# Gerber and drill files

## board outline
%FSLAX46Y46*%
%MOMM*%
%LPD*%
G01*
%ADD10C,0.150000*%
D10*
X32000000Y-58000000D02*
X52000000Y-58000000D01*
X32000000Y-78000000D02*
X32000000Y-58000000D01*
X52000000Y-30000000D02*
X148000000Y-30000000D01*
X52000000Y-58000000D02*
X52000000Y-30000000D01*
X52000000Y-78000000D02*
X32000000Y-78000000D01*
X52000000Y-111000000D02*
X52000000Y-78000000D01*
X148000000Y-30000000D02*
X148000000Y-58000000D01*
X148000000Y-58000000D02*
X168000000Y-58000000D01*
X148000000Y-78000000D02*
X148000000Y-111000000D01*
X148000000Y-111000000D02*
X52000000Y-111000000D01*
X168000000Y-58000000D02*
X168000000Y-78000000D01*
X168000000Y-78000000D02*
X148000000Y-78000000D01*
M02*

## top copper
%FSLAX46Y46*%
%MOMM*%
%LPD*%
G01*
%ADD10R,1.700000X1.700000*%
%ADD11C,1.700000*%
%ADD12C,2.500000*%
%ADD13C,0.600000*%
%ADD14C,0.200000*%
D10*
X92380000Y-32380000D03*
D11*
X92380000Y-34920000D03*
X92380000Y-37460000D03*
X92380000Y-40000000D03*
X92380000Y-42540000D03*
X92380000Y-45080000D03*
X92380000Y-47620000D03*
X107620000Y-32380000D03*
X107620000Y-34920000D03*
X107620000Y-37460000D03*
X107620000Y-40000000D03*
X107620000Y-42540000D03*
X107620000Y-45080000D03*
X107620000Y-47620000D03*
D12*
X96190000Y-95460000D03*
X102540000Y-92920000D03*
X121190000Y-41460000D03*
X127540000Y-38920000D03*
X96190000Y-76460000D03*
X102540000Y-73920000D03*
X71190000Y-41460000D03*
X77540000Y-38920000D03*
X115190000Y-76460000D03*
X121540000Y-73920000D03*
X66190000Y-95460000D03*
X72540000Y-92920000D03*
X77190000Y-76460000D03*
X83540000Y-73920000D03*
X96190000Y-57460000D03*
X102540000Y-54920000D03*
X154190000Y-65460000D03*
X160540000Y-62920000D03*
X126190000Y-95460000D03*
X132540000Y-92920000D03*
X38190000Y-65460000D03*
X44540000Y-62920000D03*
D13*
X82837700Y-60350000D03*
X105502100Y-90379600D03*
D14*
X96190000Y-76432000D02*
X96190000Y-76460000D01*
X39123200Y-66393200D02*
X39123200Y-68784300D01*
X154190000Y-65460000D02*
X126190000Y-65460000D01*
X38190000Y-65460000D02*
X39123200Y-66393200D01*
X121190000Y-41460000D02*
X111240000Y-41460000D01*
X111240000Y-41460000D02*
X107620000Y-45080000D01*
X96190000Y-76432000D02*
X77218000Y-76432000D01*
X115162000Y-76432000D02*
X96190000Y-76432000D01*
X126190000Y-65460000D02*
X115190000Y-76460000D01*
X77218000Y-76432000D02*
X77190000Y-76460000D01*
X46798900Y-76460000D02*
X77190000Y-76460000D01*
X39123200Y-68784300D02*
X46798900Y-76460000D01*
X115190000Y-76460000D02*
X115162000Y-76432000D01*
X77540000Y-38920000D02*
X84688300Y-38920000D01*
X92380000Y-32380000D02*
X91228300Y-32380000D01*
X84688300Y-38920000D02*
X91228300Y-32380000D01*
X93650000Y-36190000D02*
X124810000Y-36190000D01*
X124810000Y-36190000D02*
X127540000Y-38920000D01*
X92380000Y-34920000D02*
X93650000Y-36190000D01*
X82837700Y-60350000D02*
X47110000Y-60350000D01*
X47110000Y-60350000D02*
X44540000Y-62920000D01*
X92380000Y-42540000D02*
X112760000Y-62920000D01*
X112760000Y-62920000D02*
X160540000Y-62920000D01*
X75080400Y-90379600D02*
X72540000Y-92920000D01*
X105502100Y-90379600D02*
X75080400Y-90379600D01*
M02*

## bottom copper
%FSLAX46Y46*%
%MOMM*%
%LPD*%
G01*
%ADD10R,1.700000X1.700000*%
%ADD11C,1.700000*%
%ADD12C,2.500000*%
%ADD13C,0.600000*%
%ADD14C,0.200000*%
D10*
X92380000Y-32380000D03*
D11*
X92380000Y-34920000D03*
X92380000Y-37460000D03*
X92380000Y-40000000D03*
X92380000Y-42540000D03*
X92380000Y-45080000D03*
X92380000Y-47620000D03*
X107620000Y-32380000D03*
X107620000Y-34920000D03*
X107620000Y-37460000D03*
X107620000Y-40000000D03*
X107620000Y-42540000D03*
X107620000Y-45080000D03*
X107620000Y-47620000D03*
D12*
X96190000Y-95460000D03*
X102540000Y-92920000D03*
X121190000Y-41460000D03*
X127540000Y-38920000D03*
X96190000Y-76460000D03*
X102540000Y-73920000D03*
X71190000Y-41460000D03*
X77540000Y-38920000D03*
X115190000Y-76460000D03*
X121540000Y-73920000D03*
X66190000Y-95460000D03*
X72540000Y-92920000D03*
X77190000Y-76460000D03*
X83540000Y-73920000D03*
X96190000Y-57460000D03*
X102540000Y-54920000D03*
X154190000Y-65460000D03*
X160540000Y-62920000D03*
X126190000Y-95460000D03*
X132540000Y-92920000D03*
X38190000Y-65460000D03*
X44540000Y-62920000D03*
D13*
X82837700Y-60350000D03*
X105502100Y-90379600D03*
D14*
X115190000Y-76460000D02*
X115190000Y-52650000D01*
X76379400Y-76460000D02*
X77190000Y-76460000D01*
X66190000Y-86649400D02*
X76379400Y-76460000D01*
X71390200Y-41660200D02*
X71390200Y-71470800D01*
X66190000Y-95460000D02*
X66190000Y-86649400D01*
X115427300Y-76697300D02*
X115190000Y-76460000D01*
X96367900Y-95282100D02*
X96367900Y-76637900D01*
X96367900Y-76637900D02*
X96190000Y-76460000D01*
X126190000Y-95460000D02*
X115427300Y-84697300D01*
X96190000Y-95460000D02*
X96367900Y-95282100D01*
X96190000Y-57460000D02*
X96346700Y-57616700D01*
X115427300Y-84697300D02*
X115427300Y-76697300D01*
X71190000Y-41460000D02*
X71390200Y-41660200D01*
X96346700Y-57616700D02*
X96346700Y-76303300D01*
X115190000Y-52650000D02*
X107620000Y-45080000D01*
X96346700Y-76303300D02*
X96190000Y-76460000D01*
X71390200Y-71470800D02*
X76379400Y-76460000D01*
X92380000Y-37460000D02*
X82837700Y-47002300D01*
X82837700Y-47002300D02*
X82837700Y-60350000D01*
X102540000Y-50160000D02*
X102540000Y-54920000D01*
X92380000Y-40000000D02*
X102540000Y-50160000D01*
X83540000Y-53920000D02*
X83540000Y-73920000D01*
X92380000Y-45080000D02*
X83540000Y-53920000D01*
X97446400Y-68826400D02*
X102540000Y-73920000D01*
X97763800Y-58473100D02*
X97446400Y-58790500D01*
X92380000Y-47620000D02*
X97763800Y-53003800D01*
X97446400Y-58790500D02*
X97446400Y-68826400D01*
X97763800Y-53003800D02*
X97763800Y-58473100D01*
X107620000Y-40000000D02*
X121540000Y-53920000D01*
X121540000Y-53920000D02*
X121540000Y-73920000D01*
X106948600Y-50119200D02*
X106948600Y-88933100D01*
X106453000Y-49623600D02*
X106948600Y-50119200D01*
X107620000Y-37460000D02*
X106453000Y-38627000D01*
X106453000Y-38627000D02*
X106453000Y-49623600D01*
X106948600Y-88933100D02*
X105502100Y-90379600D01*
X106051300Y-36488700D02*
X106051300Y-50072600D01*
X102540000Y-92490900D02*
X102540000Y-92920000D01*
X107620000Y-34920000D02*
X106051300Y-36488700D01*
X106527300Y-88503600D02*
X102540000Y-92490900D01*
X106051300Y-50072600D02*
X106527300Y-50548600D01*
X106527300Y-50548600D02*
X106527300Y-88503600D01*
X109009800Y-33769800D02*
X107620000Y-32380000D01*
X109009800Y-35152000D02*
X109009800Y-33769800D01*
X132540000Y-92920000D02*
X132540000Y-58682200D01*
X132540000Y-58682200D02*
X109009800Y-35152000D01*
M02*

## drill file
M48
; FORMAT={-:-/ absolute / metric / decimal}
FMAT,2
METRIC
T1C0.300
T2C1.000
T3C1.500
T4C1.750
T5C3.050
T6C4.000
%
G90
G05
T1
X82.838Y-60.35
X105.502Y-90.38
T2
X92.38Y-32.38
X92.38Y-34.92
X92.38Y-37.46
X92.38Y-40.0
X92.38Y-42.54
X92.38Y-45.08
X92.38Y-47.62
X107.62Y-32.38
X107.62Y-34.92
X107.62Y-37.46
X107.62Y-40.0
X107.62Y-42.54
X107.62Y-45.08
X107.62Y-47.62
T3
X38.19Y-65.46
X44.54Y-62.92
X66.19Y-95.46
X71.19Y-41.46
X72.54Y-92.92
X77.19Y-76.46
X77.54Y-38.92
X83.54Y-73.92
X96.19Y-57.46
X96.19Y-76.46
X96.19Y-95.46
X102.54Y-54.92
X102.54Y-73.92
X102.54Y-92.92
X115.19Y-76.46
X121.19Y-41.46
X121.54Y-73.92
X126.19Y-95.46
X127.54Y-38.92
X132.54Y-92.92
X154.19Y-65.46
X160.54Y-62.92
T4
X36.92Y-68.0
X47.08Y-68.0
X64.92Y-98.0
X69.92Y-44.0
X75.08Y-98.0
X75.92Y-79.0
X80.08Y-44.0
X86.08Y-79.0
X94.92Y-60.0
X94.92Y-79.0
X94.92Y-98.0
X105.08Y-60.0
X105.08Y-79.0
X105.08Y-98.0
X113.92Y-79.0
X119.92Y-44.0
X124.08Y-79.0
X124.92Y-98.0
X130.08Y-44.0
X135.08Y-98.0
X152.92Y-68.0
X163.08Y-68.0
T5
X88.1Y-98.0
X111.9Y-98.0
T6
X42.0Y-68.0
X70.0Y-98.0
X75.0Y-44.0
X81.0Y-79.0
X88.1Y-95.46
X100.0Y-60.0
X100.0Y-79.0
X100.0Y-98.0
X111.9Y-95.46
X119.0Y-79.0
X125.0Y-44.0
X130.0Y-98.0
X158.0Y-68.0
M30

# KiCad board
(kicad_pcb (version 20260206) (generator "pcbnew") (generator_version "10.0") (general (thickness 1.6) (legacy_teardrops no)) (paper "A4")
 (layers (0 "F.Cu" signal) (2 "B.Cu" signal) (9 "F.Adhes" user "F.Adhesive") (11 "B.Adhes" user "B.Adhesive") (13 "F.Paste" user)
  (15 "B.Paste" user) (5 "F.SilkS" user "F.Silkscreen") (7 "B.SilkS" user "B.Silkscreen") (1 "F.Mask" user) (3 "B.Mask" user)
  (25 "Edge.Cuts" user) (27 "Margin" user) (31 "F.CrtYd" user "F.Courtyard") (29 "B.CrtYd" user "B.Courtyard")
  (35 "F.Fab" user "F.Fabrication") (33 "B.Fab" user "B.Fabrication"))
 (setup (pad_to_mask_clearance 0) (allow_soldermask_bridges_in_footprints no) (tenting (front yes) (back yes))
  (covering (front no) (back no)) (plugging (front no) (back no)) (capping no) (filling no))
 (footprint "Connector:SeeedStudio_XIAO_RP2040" (layer "F.Cu") (at 100 40)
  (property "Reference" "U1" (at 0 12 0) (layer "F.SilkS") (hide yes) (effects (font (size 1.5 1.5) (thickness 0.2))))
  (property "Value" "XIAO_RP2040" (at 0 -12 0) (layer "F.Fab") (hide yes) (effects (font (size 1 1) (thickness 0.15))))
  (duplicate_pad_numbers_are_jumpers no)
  (pad "1" thru_hole rect (at -7.62 -7.62) (size 1.7 1.7) (drill 1) (layers "*.Cu" "*.Mask") (remove_unused_layers no) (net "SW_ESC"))
  (pad "2" thru_hole circle (at -7.62 -5.08) (size 1.7 1.7) (drill 1) (layers "*.Cu" "*.Mask") (remove_unused_layers no) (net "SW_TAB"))
  (pad "3" thru_hole circle (at -7.62 -2.54) (size 1.7 1.7) (drill 1) (layers "*.Cu" "*.Mask") (remove_unused_layers no)
   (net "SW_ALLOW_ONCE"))
  (pad "4" thru_hole circle (at -7.62 0) (size 1.7 1.7) (drill 1) (layers "*.Cu" "*.Mask") (remove_unused_layers no) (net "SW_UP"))
  (pad "5" thru_hole circle (at -7.62 2.54) (size 1.7 1.7) (drill 1) (layers "*.Cu" "*.Mask") (remove_unused_layers no)
   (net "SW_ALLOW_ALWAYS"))
  (pad "6" thru_hole circle (at -7.62 5.08) (size 1.7 1.7) (drill 1) (layers "*.Cu" "*.Mask") (remove_unused_layers no) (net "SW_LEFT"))
  (pad "7" thru_hole circle (at -7.62 7.62) (size 1.7 1.7) (drill 1) (layers "*.Cu" "*.Mask") (remove_unused_layers no) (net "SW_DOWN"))
  (pad "8" thru_hole circle (at 7.62 -7.62) (size 1.7 1.7) (drill 1) (layers "*.Cu" "*.Mask") (remove_unused_layers no) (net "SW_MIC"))
  (pad "9" thru_hole circle (at 7.62 -5.08) (size 1.7 1.7) (drill 1) (layers "*.Cu" "*.Mask") (remove_unused_layers no) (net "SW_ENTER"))
  (pad "10" thru_hole circle (at 7.62 -2.54) (size 1.7 1.7) (drill 1) (layers "*.Cu" "*.Mask") (remove_unused_layers no) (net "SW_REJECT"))
  (pad "11" thru_hole circle (at 7.62 0) (size 1.7 1.7) (drill 1) (layers "*.Cu" "*.Mask") (remove_unused_layers no) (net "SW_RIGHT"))
  (pad "12" thru_hole circle (at 7.62 2.54) (size 1.7 1.7) (drill 1) (layers "*.Cu" "*.Mask") (remove_unused_layers no))
  (pad "13" thru_hole circle (at 7.62 5.08) (size 1.7 1.7) (drill 1) (layers "*.Cu" "*.Mask") (remove_unused_layers no) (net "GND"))
  (pad "14" thru_hole circle (at 7.62 7.62) (size 1.7 1.7) (drill 1) (layers "*.Cu" "*.Mask") (remove_unused_layers no)))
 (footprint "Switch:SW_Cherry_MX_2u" (layer "F.Cu") (at 100 98)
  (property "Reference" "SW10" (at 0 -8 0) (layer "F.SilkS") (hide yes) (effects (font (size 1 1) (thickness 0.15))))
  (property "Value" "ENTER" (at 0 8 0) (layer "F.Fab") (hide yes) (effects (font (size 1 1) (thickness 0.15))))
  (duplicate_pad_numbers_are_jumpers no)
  (pad "" np_thru_hole circle (at -11.9 -2.54) (size 4 4) (drill 4) (layers "*.Cu" "*.Mask"))
  (pad "" np_thru_hole circle (at -11.9 0) (size 3.05 3.05) (drill 3.05) (layers "*.Cu" "*.Mask"))
  (pad "" np_thru_hole circle (at -5.08 0) (size 1.75 1.75) (drill 1.75) (layers "*.Cu" "*.Mask"))
  (pad "" np_thru_hole circle (at 0 0) (size 4 4) (drill 4) (layers "*.Cu" "*.Mask"))
  (pad "" np_thru_hole circle (at 5.08 0) (size 1.75 1.75) (drill 1.75) (layers "*.Cu" "*.Mask"))
  (pad "" np_thru_hole circle (at 11.9 -2.54) (size 4 4) (drill 4) (layers "*.Cu" "*.Mask"))
  (pad "" np_thru_hole circle (at 11.9 0) (size 3.05 3.05) (drill 3.05) (layers "*.Cu" "*.Mask"))
  (pad "1" thru_hole circle (at -3.81 -2.54) (size 2.5 2.5) (drill 1.5) (layers "*.Cu" "*.Mask") (remove_unused_layers no) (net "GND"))
  (pad "2" thru_hole circle (at 2.54 -5.08) (size 2.5 2.5) (drill 1.5) (layers "*.Cu" "*.Mask") (remove_unused_layers no) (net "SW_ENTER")))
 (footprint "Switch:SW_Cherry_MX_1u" (layer "F.Cu") (at 125 44)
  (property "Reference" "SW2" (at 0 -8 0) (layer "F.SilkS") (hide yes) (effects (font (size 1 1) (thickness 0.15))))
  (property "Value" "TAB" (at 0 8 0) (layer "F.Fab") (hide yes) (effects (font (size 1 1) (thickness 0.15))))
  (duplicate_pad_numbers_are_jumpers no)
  (pad "" np_thru_hole circle (at -5.08 0) (size 1.75 1.75) (drill 1.75) (layers "*.Cu" "*.Mask"))
  (pad "" np_thru_hole circle (at 0 0) (size 4 4) (drill 4) (layers "*.Cu" "*.Mask"))
  (pad "" np_thru_hole circle (at 5.08 0) (size 1.75 1.75) (drill 1.75) (layers "*.Cu" "*.Mask"))
  (pad "1" thru_hole circle (at -3.81 -2.54) (size 2.5 2.5) (drill 1.5) (layers "*.Cu" "*.Mask") (remove_unused_layers no) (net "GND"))
  (pad "2" thru_hole circle (at 2.54 -5.08) (size 2.5 2.5) (drill 1.5) (layers "*.Cu" "*.Mask") (remove_unused_layers no) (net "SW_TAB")))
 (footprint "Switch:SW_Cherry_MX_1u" (layer "F.Cu") (at 100 79)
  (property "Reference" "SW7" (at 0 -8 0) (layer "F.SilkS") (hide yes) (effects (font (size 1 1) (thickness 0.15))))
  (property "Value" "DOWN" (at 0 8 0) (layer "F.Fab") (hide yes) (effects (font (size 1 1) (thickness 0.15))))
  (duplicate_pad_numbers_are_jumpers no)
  (pad "" np_thru_hole circle (at -5.08 0) (size 1.75 1.75) (drill 1.75) (layers "*.Cu" "*.Mask"))
  (pad "" np_thru_hole circle (at 0 0) (size 4 4) (drill 4) (layers "*.Cu" "*.Mask"))
  (pad "" np_thru_hole circle (at 5.08 0) (size 1.75 1.75) (drill 1.75) (layers "*.Cu" "*.Mask"))
  (pad "1" thru_hole circle (at -3.81 -2.54) (size 2.5 2.5) (drill 1.5) (layers "*.Cu" "*.Mask") (remove_unused_layers no) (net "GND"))
  (pad "2" thru_hole circle (at 2.54 -5.08) (size 2.5 2.5) (drill 1.5) (layers "*.Cu" "*.Mask") (remove_unused_layers no) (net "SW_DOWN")))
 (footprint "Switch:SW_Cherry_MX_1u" (layer "F.Cu") (at 75 44)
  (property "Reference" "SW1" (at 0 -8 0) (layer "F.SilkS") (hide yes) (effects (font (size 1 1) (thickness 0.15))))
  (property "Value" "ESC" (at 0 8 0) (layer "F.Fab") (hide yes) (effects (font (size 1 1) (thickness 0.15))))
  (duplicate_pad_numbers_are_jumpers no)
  (pad "" np_thru_hole circle (at -5.08 0) (size 1.75 1.75) (drill 1.75) (layers "*.Cu" "*.Mask"))
  (pad "" np_thru_hole circle (at 0 0) (size 4 4) (drill 4) (layers "*.Cu" "*.Mask"))
  (pad "" np_thru_hole circle (at 5.08 0) (size 1.75 1.75) (drill 1.75) (layers "*.Cu" "*.Mask"))
  (pad "1" thru_hole circle (at -3.81 -2.54) (size 2.5 2.5) (drill 1.5) (layers "*.Cu" "*.Mask") (remove_unused_layers no) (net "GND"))
  (pad "2" thru_hole circle (at 2.54 -5.08) (size 2.5 2.5) (drill 1.5) (layers "*.Cu" "*.Mask") (remove_unused_layers no) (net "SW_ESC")))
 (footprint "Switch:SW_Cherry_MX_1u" (layer "F.Cu") (at 119 79)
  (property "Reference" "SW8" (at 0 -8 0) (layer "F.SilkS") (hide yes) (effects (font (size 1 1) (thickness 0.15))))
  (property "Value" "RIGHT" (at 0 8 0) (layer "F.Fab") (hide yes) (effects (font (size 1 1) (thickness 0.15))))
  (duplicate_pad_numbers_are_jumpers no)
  (pad "" np_thru_hole circle (at -5.08 0) (size 1.75 1.75) (drill 1.75) (layers "*.Cu" "*.Mask"))
  (pad "" np_thru_hole circle (at 0 0) (size 4 4) (drill 4) (layers "*.Cu" "*.Mask"))
  (pad "" np_thru_hole circle (at 5.08 0) (size 1.75 1.75) (drill 1.75) (layers "*.Cu" "*.Mask"))
  (pad "1" thru_hole circle (at -3.81 -2.54) (size 2.5 2.5) (drill 1.5) (layers "*.Cu" "*.Mask") (remove_unused_layers no) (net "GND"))
  (pad "2" thru_hole circle (at 2.54 -5.08) (size 2.5 2.5) (drill 1.5) (layers "*.Cu" "*.Mask") (remove_unused_layers no) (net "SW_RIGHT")))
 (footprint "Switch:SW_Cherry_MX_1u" (layer "F.Cu") (at 70 98)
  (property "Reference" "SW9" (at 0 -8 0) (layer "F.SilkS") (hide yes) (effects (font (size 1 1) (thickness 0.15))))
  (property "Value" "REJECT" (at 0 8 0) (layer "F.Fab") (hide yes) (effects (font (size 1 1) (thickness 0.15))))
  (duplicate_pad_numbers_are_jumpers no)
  (pad "" np_thru_hole circle (at -5.08 0) (size 1.75 1.75) (drill 1.75) (layers "*.Cu" "*.Mask"))
  (pad "" np_thru_hole circle (at 0 0) (size 4 4) (drill 4) (layers "*.Cu" "*.Mask"))
  (pad "" np_thru_hole circle (at 5.08 0) (size 1.75 1.75) (drill 1.75) (layers "*.Cu" "*.Mask"))
  (pad "1" thru_hole circle (at -3.81 -2.54) (size 2.5 2.5) (drill 1.5) (layers "*.Cu" "*.Mask") (remove_unused_layers no) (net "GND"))
  (pad "2" thru_hole circle (at 2.54 -5.08) (size 2.5 2.5) (drill 1.5) (layers "*.Cu" "*.Mask") (remove_unused_layers no) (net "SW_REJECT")))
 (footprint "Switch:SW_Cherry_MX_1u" (layer "F.Cu") (at 81 79)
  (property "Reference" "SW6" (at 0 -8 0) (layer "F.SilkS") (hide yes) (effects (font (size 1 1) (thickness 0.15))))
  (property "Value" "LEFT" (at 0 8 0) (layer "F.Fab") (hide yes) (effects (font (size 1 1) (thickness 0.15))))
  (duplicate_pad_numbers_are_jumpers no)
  (pad "" np_thru_hole circle (at -5.08 0) (size 1.75 1.75) (drill 1.75) (layers "*.Cu" "*.Mask"))
  (pad "" np_thru_hole circle (at 0 0) (size 4 4) (drill 4) (layers "*.Cu" "*.Mask"))
  (pad "" np_thru_hole circle (at 5.08 0) (size 1.75 1.75) (drill 1.75) (layers "*.Cu" "*.Mask"))
  (pad "1" thru_hole circle (at -3.81 -2.54) (size 2.5 2.5) (drill 1.5) (layers "*.Cu" "*.Mask") (remove_unused_layers no) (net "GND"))
  (pad "2" thru_hole circle (at 2.54 -5.08) (size 2.5 2.5) (drill 1.5) (layers "*.Cu" "*.Mask") (remove_unused_layers no) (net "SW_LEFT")))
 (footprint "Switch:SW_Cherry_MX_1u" (layer "F.Cu") (at 100 60)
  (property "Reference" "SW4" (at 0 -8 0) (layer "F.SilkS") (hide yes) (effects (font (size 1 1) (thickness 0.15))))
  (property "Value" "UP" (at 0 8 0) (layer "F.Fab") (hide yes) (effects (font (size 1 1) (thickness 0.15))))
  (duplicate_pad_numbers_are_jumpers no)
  (pad "" np_thru_hole circle (at -5.08 0) (size 1.75 1.75) (drill 1.75) (layers "*.Cu" "*.Mask"))
  (pad "" np_thru_hole circle (at 0 0) (size 4 4) (drill 4) (layers "*.Cu" "*.Mask"))
  (pad "" np_thru_hole circle (at 5.08 0) (size 1.75 1.75) (drill 1.75) (layers "*.Cu" "*.Mask"))
  (pad "1" thru_hole circle (at -3.81 -2.54) (size 2.5 2.5) (drill 1.5) (layers "*.Cu" "*.Mask") (remove_unused_layers no) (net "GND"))
  (pad "2" thru_hole circle (at 2.54 -5.08) (size 2.5 2.5) (drill 1.5) (layers "*.Cu" "*.Mask") (remove_unused_layers no) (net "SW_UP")))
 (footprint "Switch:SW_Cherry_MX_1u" (layer "F.Cu") (at 158 68)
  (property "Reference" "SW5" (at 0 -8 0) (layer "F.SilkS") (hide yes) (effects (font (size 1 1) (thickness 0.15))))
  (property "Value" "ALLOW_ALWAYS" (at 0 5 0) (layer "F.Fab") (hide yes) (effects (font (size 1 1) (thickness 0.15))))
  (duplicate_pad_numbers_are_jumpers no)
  (pad "" np_thru_hole circle (at -5.08 0) (size 1.75 1.75) (drill 1.75) (layers "*.Cu" "*.Mask"))
  (pad "" np_thru_hole circle (at 0 0) (size 4 4) (drill 4) (layers "*.Cu" "*.Mask"))
  (pad "" np_thru_hole circle (at 5.08 0) (size 1.75 1.75) (drill 1.75) (layers "*.Cu" "*.Mask"))
  (pad "1" thru_hole circle (at -3.81 -2.54) (size 2.5 2.5) (drill 1.5) (layers "*.Cu" "*.Mask") (remove_unused_layers no) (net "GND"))
  (pad "2" thru_hole circle (at 2.54 -5.08) (size 2.5 2.5) (drill 1.5) (layers "*.Cu" "*.Mask") (remove_unused_layers no)
   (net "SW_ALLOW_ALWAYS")))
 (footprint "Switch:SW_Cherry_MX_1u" (layer "F.Cu") (at 130 98)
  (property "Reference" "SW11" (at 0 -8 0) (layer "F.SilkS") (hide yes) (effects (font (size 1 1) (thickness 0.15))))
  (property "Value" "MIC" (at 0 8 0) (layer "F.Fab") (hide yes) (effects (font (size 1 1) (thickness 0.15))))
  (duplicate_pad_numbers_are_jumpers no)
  (pad "" np_thru_hole circle (at -5.08 0) (size 1.75 1.75) (drill 1.75) (layers "*.Cu" "*.Mask"))
  (pad "" np_thru_hole circle (at 0 0) (size 4 4) (drill 4) (layers "*.Cu" "*.Mask"))
  (pad "" np_thru_hole circle (at 5.08 0) (size 1.75 1.75) (drill 1.75) (layers "*.Cu" "*.Mask"))
  (pad "1" thru_hole circle (at -3.81 -2.54) (size 2.5 2.5) (drill 1.5) (layers "*.Cu" "*.Mask") (remove_unused_layers no) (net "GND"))
  (pad "2" thru_hole circle (at 2.54 -5.08) (size 2.5 2.5) (drill 1.5) (layers "*.Cu" "*.Mask") (remove_unused_layers no) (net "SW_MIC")))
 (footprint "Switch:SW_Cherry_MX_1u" (layer "F.Cu") (at 42 68)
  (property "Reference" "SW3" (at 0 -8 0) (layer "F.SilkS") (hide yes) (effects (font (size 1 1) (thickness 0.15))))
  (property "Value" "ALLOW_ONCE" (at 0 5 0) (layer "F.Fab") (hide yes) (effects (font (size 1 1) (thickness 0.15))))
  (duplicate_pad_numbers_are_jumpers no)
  (pad "" np_thru_hole circle (at -5.08 0) (size 1.75 1.75) (drill 1.75) (layers "*.Cu" "*.Mask"))
  (pad "" np_thru_hole circle (at 0 0) (size 4 4) (drill 4) (layers "*.Cu" "*.Mask"))
  (pad "" np_thru_hole circle (at 5.08 0) (size 1.75 1.75) (drill 1.75) (layers "*.Cu" "*.Mask"))
  (pad "1" thru_hole circle (at -3.81 -2.54) (size 2.5 2.5) (drill 1.5) (layers "*.Cu" "*.Mask") (remove_unused_layers no) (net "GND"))
  (pad "2" thru_hole circle (at 2.54 -5.08) (size 2.5 2.5) (drill 1.5) (layers "*.Cu" "*.Mask") (remove_unused_layers no)
   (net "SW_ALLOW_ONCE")))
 (gr_line (start 32 58) (end 52 58) (stroke (width 0.15) (type solid)) (layer "Edge.Cuts"))
 (gr_line (start 32 78) (end 32 58) (stroke (width 0.15) (type solid)) (layer "Edge.Cuts"))
 (gr_line (start 52 30) (end 148 30) (stroke (width 0.15) (type solid)) (layer "Edge.Cuts"))
 (gr_line (start 52 58) (end 52 30) (stroke (width 0.15) (type solid)) (layer "Edge.Cuts"))
 (gr_line (start 52 78) (end 32 78) (stroke (width 0.15) (type solid)) (layer "Edge.Cuts"))
 (gr_line (start 52 111) (end 52 78) (stroke (width 0.15) (type solid)) (layer "Edge.Cuts"))
 (gr_line (start 148 30) (end 148 58) (stroke (width 0.15) (type solid)) (layer "Edge.Cuts"))
 (gr_line (start 148 58) (end 168 58) (stroke (width 0.15) (type solid)) (layer "Edge.Cuts"))
 (gr_line (start 148 78) (end 148 111) (stroke (width 0.15) (type solid)) (layer "Edge.Cuts"))
 (gr_line (start 148 111) (end 52 111) (stroke (width 0.15) (type solid)) (layer "Edge.Cuts"))
 (gr_line (start 168 58) (end 168 78) (stroke (width 0.15) (type solid)) (layer "Edge.Cuts"))
 (gr_line (start 168 78) (end 148 78) (stroke (width 0.15) (type solid)) (layer "Edge.Cuts"))
 (segment (start 96.19 76.432) (end 96.19 76.46) (width 0.2) (layer "F.Cu") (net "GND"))
 (segment (start 39.1232 66.3932) (end 39.1232 68.7843) (width 0.2) (layer "F.Cu") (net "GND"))
 (segment (start 154.19 65.46) (end 126.19 65.46) (width 0.2) (layer "F.Cu") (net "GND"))
 (segment (start 38.19 65.46) (end 39.1232 66.3932) (width 0.2) (layer "F.Cu") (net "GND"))
 (segment (start 121.19 41.46) (end 111.24 41.46) (width 0.2) (layer "F.Cu") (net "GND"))
 (segment (start 111.24 41.46) (end 107.62 45.08) (width 0.2) (layer "F.Cu") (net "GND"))
 (segment (start 96.19 76.432) (end 77.218 76.432) (width 0.2) (layer "F.Cu") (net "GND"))
 (segment (start 115.162 76.432) (end 96.19 76.432) (width 0.2) (layer "F.Cu") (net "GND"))
 (segment (start 126.19 65.46) (end 115.19 76.46) (width 0.2) (layer "F.Cu") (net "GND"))
 (segment (start 77.218 76.432) (end 77.19 76.46) (width 0.2) (layer "F.Cu") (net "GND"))
 (segment (start 46.7989 76.46) (end 77.19 76.46) (width 0.2) (layer "F.Cu") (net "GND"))
 (segment (start 39.1232 68.7843) (end 46.7989 76.46) (width 0.2) (layer "F.Cu") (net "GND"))
 (segment (start 115.19 76.46) (end 115.162 76.432) (width 0.2) (layer "F.Cu") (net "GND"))
 (segment (start 115.19 76.46) (end 115.19 52.65) (width 0.2) (layer "B.Cu") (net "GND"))
 (segment (start 76.3794 76.46) (end 77.19 76.46) (width 0.2) (layer "B.Cu") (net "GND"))
 (segment (start 66.19 86.6494) (end 76.3794 76.46) (width 0.2) (layer "B.Cu") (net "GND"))
 (segment (start 71.3902 41.6602) (end 71.3902 71.4708) (width 0.2) (layer "B.Cu") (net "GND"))
 (segment (start 66.19 95.46) (end 66.19 86.6494) (width 0.2) (layer "B.Cu") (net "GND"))
 (segment (start 115.4273 76.6973) (end 115.19 76.46) (width 0.2) (layer "B.Cu") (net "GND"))
 (segment (start 96.3679 95.2821) (end 96.3679 76.6379) (width 0.2) (layer "B.Cu") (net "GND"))
 (segment (start 96.3679 76.6379) (end 96.19 76.46) (width 0.2) (layer "B.Cu") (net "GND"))
 (segment (start 126.19 95.46) (end 115.4273 84.6973) (width 0.2) (layer "B.Cu") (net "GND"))
 (segment (start 96.19 95.46) (end 96.3679 95.2821) (width 0.2) (layer "B.Cu") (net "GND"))
 (segment (start 96.19 57.46) (end 96.3467 57.6167) (width 0.2) (layer "B.Cu") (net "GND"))
 (segment (start 115.4273 84.6973) (end 115.4273 76.6973) (width 0.2) (layer "B.Cu") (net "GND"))
 (segment (start 71.19 41.46) (end 71.3902 41.6602) (width 0.2) (layer "B.Cu") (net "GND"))
 (segment (start 96.3467 57.6167) (end 96.3467 76.3033) (width 0.2) (layer "B.Cu") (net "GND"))
 (segment (start 115.19 52.65) (end 107.62 45.08) (width 0.2) (layer "B.Cu") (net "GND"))
 (segment (start 96.3467 76.3033) (end 96.19 76.46) (width 0.2) (layer "B.Cu") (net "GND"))
 (segment (start 71.3902 71.4708) (end 76.3794 76.46) (width 0.2) (layer "B.Cu") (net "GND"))
 (segment (start 77.54 38.92) (end 84.6883 38.92) (width 0.2) (layer "F.Cu") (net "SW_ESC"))
 (segment (start 92.38 32.38) (end 91.2283 32.38) (width 0.2) (layer "F.Cu") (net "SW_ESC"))
 (segment (start 84.6883 38.92) (end 91.2283 32.38) (width 0.2) (layer "F.Cu") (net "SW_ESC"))
 (segment (start 93.65 36.19) (end 124.81 36.19) (width 0.2) (layer "F.Cu") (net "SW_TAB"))
 (segment (start 124.81 36.19) (end 127.54 38.92) (width 0.2) (layer "F.Cu") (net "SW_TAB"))
 (segment (start 92.38 34.92) (end 93.65 36.19) (width 0.2) (layer "F.Cu") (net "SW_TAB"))
 (segment (start 82.8377 60.35) (end 47.11 60.35) (width 0.2) (layer "F.Cu") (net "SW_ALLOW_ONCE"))
 (segment (start 47.11 60.35) (end 44.54 62.92) (width 0.2) (layer "F.Cu") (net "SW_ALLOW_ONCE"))
 (via (at 82.8377 60.35) (size 0.6) (drill 0.3) (layers "F.Cu" "B.Cu") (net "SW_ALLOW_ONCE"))
 (segment (start 92.38 37.46) (end 82.8377 47.0023) (width 0.2) (layer "B.Cu") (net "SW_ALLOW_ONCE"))
 (segment (start 82.8377 47.0023) (end 82.8377 60.35) (width 0.2) (layer "B.Cu") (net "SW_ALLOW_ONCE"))
 (segment (start 102.54 50.16) (end 102.54 54.92) (width 0.2) (layer "B.Cu") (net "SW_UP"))
 (segment (start 92.38 40) (end 102.54 50.16) (width 0.2) (layer "B.Cu") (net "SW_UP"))
 (segment (start 92.38 42.54) (end 112.76 62.92) (width 0.2) (layer "F.Cu") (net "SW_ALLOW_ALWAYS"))
 (segment (start 112.76 62.92) (end 160.54 62.92) (width 0.2) (layer "F.Cu") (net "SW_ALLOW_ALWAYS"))
 (segment (start 83.54 53.92) (end 83.54 73.92) (width 0.2) (layer "B.Cu") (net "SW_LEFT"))
 (segment (start 92.38 45.08) (end 83.54 53.92) (width 0.2) (layer "B.Cu") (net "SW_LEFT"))
 (segment (start 97.4464 68.8264) (end 102.54 73.92) (width 0.2) (layer "B.Cu") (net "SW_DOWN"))
 (segment (start 97.7638 58.4731) (end 97.4464 58.7905) (width 0.2) (layer "B.Cu") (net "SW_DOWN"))
 (segment (start 92.38 47.62) (end 97.7638 53.0038) (width 0.2) (layer "B.Cu") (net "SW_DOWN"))
 (segment (start 97.4464 58.7905) (end 97.4464 68.8264) (width 0.2) (layer "B.Cu") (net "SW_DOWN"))
 (segment (start 97.7638 53.0038) (end 97.7638 58.4731) (width 0.2) (layer "B.Cu") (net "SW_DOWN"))
 (segment (start 107.62 40) (end 121.54 53.92) (width 0.2) (layer "B.Cu") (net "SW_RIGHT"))
 (segment (start 121.54 53.92) (end 121.54 73.92) (width 0.2) (layer "B.Cu") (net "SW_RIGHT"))
 (segment (start 75.0804 90.3796) (end 72.54 92.92) (width 0.2) (layer "F.Cu") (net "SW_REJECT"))
 (segment (start 105.5021 90.3796) (end 75.0804 90.3796) (width 0.2) (layer "F.Cu") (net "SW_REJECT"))
 (via (at 105.5021 90.3796) (size 0.6) (drill 0.3) (layers "F.Cu" "B.Cu") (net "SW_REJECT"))
 (segment (start 106.9486 50.1192) (end 106.9486 88.9331) (width 0.2) (layer "B.Cu") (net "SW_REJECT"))
 (segment (start 106.453 49.6236) (end 106.9486 50.1192) (width 0.2) (layer "B.Cu") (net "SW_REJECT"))
 (segment (start 107.62 37.46) (end 106.453 38.627) (width 0.2) (layer "B.Cu") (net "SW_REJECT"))
 (segment (start 106.453 38.627) (end 106.453 49.6236) (width 0.2) (layer "B.Cu") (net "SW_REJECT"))
 (segment (start 106.9486 88.9331) (end 105.5021 90.3796) (width 0.2) (layer "B.Cu") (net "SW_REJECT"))
 (segment (start 106.0513 36.4887) (end 106.0513 50.0726) (width 0.2) (layer "B.Cu") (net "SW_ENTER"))
 (segment (start 102.54 92.4909) (end 102.54 92.92) (width 0.2) (layer "B.Cu") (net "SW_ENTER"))
 (segment (start 107.62 34.92) (end 106.0513 36.4887) (width 0.2) (layer "B.Cu") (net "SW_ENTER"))
 (segment (start 106.5273 88.5036) (end 102.54 92.4909) (width 0.2) (layer "B.Cu") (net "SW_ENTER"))
 (segment (start 106.0513 50.0726) (end 106.5273 50.5486) (width 0.2) (layer "B.Cu") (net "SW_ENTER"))
 (segment (start 106.5273 50.5486) (end 106.5273 88.5036) (width 0.2) (layer "B.Cu") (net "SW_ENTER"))
 (segment (start 109.0098 33.7698) (end 107.62 32.38) (width 0.2) (layer "B.Cu") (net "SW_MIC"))
 (segment (start 109.0098 35.152) (end 109.0098 33.7698) (width 0.2) (layer "B.Cu") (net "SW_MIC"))
 (segment (start 132.54 92.92) (end 132.54 58.6822) (width 0.2) (layer "B.Cu") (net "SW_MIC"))
 (segment (start 132.54 58.6822) (end 109.0098 35.152) (width 0.2) (layer "B.Cu") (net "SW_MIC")))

